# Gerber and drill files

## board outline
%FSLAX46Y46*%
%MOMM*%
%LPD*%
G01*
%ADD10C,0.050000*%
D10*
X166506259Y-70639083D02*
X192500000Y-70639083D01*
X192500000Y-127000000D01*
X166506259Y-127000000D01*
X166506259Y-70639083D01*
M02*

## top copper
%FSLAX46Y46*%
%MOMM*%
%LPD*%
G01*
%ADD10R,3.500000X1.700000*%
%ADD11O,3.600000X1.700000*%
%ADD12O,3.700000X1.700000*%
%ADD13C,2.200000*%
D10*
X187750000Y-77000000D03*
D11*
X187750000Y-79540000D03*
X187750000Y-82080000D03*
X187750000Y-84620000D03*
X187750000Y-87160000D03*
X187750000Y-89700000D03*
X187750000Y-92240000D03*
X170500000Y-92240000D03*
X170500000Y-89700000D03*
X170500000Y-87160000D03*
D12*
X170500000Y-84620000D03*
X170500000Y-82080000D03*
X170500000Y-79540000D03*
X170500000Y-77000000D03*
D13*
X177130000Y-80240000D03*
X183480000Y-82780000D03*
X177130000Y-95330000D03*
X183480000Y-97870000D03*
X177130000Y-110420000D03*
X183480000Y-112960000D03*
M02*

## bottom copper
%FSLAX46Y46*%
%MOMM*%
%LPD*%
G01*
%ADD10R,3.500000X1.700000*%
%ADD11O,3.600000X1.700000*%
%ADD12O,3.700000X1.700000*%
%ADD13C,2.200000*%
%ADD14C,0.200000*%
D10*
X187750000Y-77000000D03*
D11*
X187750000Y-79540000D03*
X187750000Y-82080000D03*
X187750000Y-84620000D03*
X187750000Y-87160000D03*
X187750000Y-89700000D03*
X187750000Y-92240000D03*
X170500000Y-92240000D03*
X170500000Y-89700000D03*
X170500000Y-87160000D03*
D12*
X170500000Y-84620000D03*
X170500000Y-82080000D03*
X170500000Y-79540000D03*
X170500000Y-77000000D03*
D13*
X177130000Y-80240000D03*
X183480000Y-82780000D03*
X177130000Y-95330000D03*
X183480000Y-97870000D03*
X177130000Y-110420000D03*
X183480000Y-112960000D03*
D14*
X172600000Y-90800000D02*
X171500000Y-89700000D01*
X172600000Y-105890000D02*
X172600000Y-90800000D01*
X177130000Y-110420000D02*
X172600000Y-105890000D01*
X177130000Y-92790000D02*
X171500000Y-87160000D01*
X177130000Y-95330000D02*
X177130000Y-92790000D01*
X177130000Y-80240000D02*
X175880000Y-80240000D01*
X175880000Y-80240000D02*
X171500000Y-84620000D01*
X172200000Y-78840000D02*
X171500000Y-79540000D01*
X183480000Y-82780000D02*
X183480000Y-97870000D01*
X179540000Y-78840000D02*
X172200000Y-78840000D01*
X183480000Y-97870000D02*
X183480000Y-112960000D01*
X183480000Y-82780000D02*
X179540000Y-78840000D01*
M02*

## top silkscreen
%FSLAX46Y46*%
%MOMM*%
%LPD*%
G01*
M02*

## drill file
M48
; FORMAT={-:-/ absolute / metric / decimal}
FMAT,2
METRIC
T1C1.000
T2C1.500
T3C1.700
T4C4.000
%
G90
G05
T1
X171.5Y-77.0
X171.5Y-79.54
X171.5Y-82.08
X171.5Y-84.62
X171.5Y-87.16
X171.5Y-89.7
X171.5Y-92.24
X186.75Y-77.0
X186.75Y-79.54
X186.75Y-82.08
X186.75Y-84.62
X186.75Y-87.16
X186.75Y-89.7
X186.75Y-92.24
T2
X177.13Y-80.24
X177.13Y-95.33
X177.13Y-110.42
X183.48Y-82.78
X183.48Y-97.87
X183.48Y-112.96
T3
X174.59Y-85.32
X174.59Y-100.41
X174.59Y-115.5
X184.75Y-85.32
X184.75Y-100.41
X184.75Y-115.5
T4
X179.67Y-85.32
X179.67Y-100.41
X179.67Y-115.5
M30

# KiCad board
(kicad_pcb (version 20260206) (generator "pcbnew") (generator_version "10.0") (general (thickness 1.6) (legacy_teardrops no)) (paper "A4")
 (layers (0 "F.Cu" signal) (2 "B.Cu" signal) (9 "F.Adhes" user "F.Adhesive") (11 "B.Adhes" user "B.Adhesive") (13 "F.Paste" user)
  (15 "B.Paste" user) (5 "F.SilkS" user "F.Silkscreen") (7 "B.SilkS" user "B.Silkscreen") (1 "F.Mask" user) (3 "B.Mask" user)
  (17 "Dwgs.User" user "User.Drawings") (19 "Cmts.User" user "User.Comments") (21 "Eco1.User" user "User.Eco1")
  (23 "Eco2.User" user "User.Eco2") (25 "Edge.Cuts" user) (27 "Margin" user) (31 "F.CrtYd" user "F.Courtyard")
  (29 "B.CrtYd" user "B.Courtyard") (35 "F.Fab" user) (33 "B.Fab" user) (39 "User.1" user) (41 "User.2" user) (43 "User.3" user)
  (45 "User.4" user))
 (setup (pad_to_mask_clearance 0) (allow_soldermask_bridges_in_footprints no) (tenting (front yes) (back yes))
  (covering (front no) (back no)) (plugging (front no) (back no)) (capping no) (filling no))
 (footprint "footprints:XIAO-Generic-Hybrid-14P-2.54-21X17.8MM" (layer "B.Cu") (at 179.125 84.62 180)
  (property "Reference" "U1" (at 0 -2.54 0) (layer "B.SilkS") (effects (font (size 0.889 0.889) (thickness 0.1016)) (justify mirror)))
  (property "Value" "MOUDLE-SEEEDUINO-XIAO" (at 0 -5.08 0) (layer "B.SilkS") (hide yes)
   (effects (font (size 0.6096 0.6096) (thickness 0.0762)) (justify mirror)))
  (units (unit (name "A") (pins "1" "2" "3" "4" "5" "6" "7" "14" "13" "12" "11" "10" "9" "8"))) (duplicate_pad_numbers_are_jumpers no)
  (pad "1" thru_hole rect (at -7.625 7.62 180) (size 3.5 1.7) (drill 1 (offset -1 0)) (layers "*.Cu" "*.Mask") (remove_unused_layers no)
   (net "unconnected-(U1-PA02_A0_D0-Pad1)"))
  (pad "2" thru_hole oval (at -7.625 5.08 180) (size 3.6 1.7) (drill 1 (offset -1 0)) (layers "*.Cu" "*.Mask") (remove_unused_layers no)
   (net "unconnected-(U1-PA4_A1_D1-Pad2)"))
  (pad "3" thru_hole oval (at -7.625 2.54 180) (size 3.6 1.7) (drill 1 (offset -1 0)) (layers "*.Cu" "*.Mask") (remove_unused_layers no)
   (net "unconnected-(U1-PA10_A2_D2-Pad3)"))
  (pad "4" thru_hole oval (at -7.625 0 180) (size 3.6 1.7) (drill 1 (offset -1 0)) (layers "*.Cu" "*.Mask") (remove_unused_layers no)
   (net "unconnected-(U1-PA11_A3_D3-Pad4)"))
  (pad "5" thru_hole oval (at -7.625 -2.54 180) (size 3.6 1.7) (drill 1 (offset -1 0)) (layers "*.Cu" "*.Mask") (remove_unused_layers no)
   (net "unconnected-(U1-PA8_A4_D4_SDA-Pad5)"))
  (pad "6" thru_hole oval (at -7.625 -5.08) (size 3.6 1.7) (drill 1 (offset 1 0)) (layers "*.Cu" "*.Mask") (remove_unused_layers no)
   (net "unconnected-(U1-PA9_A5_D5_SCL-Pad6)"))
  (pad "7" thru_hole oval (at -7.625 -7.62 180) (size 3.6 1.7) (drill 1 (offset -1 0)) (layers "*.Cu" "*.Mask") (remove_unused_layers no)
   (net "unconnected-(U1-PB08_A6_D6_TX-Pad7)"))
  (pad "8" thru_hole oval (at 7.625 -7.62 180) (size 3.6 1.7) (drill 1 (offset 1 0)) (layers "*.Cu" "*.Mask") (remove_unused_layers no)
   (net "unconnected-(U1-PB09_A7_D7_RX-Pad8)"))
  (pad "9" thru_hole oval (at 7.625 -5.08 180) (size 3.6 1.7) (drill 1 (offset 1 0)) (layers "*.Cu" "*.Mask") (remove_unused_layers no)
   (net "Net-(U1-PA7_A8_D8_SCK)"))
  (pad "10" thru_hole oval (at 7.625 -2.54 180) (size 3.6 1.7) (drill 1 (offset 1 0)) (layers "*.Cu" "*.Mask") (remove_unused_layers no)
   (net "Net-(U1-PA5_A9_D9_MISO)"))
  (pad "11" thru_hole oval (at 7.625 0 180) (size 3.7 1.7) (drill 1 (offset 1 0)) (layers "*.Cu" "*.Mask") (remove_unused_layers no)
   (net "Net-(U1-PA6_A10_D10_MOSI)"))
  (pad "12" thru_hole oval (at 7.625 2.54 180) (size 3.7 1.7) (drill 1 (offset 1 0)) (layers "*.Cu" "*.Mask") (remove_unused_layers no)
   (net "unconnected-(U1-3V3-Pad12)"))
  (pad "13" thru_hole oval (at 7.625 5.08 180) (size 3.7 1.7) (drill 1 (offset 1 0)) (layers "*.Cu" "*.Mask") (remove_unused_layers no)
   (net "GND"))
  (pad "14" thru_hole oval (at 7.625 7.62 180) (size 3.7 1.7) (drill 1 (offset 1 0)) (layers "*.Cu" "*.Mask") (remove_unused_layers no)
   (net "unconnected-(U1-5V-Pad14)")))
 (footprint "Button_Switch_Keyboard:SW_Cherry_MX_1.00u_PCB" (layer "B.Cu") (at 177.13 80.24 180)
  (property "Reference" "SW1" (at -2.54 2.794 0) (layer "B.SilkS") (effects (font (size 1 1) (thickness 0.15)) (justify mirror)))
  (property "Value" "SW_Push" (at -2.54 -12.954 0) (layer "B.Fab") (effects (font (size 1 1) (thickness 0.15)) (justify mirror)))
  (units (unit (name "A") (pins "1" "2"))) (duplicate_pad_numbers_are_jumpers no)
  (pad "" np_thru_hole circle (at -7.62 -5.08 180) (size 1.7 1.7) (drill 1.7) (layers "*.Cu" "*.Mask"))
  (pad "" np_thru_hole circle (at -2.54 -5.08 180) (size 4 4) (drill 4) (layers "*.Cu" "*.Mask"))
  (pad "" np_thru_hole circle (at 2.54 -5.08 180) (size 1.7 1.7) (drill 1.7) (layers "*.Cu" "*.Mask"))
  (pad "1" thru_hole circle (at 0 0 180) (size 2.2 2.2) (drill 1.5) (layers "*.Cu" "*.Mask") (remove_unused_layers no)
   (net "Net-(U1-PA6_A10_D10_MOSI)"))
  (pad "2" thru_hole circle (at -6.35 -2.54 180) (size 2.2 2.2) (drill 1.5) (layers "*.Cu" "*.Mask") (remove_unused_layers no) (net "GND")))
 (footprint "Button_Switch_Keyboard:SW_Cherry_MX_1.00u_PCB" (layer "B.Cu") (at 177.13 95.33 180)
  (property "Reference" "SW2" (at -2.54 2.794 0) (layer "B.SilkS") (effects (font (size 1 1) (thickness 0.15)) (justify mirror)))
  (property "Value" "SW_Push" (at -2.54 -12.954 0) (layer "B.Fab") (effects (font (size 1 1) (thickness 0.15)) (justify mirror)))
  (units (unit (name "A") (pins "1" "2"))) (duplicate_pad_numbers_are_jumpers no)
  (pad "" np_thru_hole circle (at -7.62 -5.08 180) (size 1.7 1.7) (drill 1.7) (layers "*.Cu" "*.Mask"))
  (pad "" np_thru_hole circle (at -2.54 -5.08 180) (size 4 4) (drill 4) (layers "*.Cu" "*.Mask"))
  (pad "" np_thru_hole circle (at 2.54 -5.08 180) (size 1.7 1.7) (drill 1.7) (layers "*.Cu" "*.Mask"))
  (pad "1" thru_hole circle (at 0 0 180) (size 2.2 2.2) (drill 1.5) (layers "*.Cu" "*.Mask") (remove_unused_layers no)
   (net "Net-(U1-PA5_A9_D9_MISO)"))
  (pad "2" thru_hole circle (at -6.35 -2.54 180) (size 2.2 2.2) (drill 1.5) (layers "*.Cu" "*.Mask") (remove_unused_layers no) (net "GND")))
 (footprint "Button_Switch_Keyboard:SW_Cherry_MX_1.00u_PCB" (layer "B.Cu") (at 177.13 110.42 180)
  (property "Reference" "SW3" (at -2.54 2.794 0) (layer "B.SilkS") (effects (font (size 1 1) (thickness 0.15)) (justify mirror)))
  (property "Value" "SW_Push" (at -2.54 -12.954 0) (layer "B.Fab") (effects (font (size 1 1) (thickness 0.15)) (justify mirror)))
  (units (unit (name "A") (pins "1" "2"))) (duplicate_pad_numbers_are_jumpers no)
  (pad "" np_thru_hole circle (at -7.62 -5.08 180) (size 1.7 1.7) (drill 1.7) (layers "*.Cu" "*.Mask"))
  (pad "" np_thru_hole circle (at -2.54 -5.08 180) (size 4 4) (drill 4) (layers "*.Cu" "*.Mask"))
  (pad "" np_thru_hole circle (at 2.54 -5.08 180) (size 1.7 1.7) (drill 1.7) (layers "*.Cu" "*.Mask"))
  (pad "1" thru_hole circle (at 0 0 180) (size 2.2 2.2) (drill 1.5) (layers "*.Cu" "*.Mask") (remove_unused_layers no)
   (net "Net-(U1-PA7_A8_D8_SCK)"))
  (pad "2" thru_hole circle (at -6.35 -2.54 180) (size 2.2 2.2) (drill 1.5) (layers "*.Cu" "*.Mask") (remove_unused_layers no) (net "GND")))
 (gr_rect (start 166.506259 70.639083) (end 192.5 127) (stroke (width 0.05) (type default)) (fill no) (layer "Edge.Cuts"))
 (segment (start 172.6 90.8) (end 171.5 89.7) (width 0.2) (layer "B.Cu") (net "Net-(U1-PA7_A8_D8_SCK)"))
 (segment (start 172.6 105.89) (end 172.6 90.8) (width 0.2) (layer "B.Cu") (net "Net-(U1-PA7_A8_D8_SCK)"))
 (segment (start 177.13 110.42) (end 172.6 105.89) (width 0.2) (layer "B.Cu") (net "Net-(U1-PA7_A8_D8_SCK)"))
 (segment (start 177.13 92.79) (end 171.5 87.16) (width 0.2) (layer "B.Cu") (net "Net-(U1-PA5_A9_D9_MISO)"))
 (segment (start 177.13 95.33) (end 177.13 92.79) (width 0.2) (layer "B.Cu") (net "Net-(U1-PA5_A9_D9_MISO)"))
 (segment (start 177.13 80.24) (end 175.88 80.24) (width 0.2) (layer "B.Cu") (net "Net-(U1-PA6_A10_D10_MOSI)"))
 (segment (start 175.88 80.24) (end 171.5 84.62) (width 0.2) (layer "B.Cu") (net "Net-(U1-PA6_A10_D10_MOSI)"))
 (segment (start 172.2 78.84) (end 171.5 79.54) (width 0.2) (layer "B.Cu") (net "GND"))
 (segment (start 183.48 82.78) (end 183.48 97.87) (width 0.2) (layer "B.Cu") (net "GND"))
 (segment (start 179.54 78.84) (end 172.2 78.84) (width 0.2) (layer "B.Cu") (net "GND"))
 (segment (start 183.48 97.87) (end 183.48 112.96) (width 0.2) (layer "B.Cu") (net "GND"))
 (segment (start 183.48 82.78) (end 179.54 78.84) (width 0.2) (layer "B.Cu") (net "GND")))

